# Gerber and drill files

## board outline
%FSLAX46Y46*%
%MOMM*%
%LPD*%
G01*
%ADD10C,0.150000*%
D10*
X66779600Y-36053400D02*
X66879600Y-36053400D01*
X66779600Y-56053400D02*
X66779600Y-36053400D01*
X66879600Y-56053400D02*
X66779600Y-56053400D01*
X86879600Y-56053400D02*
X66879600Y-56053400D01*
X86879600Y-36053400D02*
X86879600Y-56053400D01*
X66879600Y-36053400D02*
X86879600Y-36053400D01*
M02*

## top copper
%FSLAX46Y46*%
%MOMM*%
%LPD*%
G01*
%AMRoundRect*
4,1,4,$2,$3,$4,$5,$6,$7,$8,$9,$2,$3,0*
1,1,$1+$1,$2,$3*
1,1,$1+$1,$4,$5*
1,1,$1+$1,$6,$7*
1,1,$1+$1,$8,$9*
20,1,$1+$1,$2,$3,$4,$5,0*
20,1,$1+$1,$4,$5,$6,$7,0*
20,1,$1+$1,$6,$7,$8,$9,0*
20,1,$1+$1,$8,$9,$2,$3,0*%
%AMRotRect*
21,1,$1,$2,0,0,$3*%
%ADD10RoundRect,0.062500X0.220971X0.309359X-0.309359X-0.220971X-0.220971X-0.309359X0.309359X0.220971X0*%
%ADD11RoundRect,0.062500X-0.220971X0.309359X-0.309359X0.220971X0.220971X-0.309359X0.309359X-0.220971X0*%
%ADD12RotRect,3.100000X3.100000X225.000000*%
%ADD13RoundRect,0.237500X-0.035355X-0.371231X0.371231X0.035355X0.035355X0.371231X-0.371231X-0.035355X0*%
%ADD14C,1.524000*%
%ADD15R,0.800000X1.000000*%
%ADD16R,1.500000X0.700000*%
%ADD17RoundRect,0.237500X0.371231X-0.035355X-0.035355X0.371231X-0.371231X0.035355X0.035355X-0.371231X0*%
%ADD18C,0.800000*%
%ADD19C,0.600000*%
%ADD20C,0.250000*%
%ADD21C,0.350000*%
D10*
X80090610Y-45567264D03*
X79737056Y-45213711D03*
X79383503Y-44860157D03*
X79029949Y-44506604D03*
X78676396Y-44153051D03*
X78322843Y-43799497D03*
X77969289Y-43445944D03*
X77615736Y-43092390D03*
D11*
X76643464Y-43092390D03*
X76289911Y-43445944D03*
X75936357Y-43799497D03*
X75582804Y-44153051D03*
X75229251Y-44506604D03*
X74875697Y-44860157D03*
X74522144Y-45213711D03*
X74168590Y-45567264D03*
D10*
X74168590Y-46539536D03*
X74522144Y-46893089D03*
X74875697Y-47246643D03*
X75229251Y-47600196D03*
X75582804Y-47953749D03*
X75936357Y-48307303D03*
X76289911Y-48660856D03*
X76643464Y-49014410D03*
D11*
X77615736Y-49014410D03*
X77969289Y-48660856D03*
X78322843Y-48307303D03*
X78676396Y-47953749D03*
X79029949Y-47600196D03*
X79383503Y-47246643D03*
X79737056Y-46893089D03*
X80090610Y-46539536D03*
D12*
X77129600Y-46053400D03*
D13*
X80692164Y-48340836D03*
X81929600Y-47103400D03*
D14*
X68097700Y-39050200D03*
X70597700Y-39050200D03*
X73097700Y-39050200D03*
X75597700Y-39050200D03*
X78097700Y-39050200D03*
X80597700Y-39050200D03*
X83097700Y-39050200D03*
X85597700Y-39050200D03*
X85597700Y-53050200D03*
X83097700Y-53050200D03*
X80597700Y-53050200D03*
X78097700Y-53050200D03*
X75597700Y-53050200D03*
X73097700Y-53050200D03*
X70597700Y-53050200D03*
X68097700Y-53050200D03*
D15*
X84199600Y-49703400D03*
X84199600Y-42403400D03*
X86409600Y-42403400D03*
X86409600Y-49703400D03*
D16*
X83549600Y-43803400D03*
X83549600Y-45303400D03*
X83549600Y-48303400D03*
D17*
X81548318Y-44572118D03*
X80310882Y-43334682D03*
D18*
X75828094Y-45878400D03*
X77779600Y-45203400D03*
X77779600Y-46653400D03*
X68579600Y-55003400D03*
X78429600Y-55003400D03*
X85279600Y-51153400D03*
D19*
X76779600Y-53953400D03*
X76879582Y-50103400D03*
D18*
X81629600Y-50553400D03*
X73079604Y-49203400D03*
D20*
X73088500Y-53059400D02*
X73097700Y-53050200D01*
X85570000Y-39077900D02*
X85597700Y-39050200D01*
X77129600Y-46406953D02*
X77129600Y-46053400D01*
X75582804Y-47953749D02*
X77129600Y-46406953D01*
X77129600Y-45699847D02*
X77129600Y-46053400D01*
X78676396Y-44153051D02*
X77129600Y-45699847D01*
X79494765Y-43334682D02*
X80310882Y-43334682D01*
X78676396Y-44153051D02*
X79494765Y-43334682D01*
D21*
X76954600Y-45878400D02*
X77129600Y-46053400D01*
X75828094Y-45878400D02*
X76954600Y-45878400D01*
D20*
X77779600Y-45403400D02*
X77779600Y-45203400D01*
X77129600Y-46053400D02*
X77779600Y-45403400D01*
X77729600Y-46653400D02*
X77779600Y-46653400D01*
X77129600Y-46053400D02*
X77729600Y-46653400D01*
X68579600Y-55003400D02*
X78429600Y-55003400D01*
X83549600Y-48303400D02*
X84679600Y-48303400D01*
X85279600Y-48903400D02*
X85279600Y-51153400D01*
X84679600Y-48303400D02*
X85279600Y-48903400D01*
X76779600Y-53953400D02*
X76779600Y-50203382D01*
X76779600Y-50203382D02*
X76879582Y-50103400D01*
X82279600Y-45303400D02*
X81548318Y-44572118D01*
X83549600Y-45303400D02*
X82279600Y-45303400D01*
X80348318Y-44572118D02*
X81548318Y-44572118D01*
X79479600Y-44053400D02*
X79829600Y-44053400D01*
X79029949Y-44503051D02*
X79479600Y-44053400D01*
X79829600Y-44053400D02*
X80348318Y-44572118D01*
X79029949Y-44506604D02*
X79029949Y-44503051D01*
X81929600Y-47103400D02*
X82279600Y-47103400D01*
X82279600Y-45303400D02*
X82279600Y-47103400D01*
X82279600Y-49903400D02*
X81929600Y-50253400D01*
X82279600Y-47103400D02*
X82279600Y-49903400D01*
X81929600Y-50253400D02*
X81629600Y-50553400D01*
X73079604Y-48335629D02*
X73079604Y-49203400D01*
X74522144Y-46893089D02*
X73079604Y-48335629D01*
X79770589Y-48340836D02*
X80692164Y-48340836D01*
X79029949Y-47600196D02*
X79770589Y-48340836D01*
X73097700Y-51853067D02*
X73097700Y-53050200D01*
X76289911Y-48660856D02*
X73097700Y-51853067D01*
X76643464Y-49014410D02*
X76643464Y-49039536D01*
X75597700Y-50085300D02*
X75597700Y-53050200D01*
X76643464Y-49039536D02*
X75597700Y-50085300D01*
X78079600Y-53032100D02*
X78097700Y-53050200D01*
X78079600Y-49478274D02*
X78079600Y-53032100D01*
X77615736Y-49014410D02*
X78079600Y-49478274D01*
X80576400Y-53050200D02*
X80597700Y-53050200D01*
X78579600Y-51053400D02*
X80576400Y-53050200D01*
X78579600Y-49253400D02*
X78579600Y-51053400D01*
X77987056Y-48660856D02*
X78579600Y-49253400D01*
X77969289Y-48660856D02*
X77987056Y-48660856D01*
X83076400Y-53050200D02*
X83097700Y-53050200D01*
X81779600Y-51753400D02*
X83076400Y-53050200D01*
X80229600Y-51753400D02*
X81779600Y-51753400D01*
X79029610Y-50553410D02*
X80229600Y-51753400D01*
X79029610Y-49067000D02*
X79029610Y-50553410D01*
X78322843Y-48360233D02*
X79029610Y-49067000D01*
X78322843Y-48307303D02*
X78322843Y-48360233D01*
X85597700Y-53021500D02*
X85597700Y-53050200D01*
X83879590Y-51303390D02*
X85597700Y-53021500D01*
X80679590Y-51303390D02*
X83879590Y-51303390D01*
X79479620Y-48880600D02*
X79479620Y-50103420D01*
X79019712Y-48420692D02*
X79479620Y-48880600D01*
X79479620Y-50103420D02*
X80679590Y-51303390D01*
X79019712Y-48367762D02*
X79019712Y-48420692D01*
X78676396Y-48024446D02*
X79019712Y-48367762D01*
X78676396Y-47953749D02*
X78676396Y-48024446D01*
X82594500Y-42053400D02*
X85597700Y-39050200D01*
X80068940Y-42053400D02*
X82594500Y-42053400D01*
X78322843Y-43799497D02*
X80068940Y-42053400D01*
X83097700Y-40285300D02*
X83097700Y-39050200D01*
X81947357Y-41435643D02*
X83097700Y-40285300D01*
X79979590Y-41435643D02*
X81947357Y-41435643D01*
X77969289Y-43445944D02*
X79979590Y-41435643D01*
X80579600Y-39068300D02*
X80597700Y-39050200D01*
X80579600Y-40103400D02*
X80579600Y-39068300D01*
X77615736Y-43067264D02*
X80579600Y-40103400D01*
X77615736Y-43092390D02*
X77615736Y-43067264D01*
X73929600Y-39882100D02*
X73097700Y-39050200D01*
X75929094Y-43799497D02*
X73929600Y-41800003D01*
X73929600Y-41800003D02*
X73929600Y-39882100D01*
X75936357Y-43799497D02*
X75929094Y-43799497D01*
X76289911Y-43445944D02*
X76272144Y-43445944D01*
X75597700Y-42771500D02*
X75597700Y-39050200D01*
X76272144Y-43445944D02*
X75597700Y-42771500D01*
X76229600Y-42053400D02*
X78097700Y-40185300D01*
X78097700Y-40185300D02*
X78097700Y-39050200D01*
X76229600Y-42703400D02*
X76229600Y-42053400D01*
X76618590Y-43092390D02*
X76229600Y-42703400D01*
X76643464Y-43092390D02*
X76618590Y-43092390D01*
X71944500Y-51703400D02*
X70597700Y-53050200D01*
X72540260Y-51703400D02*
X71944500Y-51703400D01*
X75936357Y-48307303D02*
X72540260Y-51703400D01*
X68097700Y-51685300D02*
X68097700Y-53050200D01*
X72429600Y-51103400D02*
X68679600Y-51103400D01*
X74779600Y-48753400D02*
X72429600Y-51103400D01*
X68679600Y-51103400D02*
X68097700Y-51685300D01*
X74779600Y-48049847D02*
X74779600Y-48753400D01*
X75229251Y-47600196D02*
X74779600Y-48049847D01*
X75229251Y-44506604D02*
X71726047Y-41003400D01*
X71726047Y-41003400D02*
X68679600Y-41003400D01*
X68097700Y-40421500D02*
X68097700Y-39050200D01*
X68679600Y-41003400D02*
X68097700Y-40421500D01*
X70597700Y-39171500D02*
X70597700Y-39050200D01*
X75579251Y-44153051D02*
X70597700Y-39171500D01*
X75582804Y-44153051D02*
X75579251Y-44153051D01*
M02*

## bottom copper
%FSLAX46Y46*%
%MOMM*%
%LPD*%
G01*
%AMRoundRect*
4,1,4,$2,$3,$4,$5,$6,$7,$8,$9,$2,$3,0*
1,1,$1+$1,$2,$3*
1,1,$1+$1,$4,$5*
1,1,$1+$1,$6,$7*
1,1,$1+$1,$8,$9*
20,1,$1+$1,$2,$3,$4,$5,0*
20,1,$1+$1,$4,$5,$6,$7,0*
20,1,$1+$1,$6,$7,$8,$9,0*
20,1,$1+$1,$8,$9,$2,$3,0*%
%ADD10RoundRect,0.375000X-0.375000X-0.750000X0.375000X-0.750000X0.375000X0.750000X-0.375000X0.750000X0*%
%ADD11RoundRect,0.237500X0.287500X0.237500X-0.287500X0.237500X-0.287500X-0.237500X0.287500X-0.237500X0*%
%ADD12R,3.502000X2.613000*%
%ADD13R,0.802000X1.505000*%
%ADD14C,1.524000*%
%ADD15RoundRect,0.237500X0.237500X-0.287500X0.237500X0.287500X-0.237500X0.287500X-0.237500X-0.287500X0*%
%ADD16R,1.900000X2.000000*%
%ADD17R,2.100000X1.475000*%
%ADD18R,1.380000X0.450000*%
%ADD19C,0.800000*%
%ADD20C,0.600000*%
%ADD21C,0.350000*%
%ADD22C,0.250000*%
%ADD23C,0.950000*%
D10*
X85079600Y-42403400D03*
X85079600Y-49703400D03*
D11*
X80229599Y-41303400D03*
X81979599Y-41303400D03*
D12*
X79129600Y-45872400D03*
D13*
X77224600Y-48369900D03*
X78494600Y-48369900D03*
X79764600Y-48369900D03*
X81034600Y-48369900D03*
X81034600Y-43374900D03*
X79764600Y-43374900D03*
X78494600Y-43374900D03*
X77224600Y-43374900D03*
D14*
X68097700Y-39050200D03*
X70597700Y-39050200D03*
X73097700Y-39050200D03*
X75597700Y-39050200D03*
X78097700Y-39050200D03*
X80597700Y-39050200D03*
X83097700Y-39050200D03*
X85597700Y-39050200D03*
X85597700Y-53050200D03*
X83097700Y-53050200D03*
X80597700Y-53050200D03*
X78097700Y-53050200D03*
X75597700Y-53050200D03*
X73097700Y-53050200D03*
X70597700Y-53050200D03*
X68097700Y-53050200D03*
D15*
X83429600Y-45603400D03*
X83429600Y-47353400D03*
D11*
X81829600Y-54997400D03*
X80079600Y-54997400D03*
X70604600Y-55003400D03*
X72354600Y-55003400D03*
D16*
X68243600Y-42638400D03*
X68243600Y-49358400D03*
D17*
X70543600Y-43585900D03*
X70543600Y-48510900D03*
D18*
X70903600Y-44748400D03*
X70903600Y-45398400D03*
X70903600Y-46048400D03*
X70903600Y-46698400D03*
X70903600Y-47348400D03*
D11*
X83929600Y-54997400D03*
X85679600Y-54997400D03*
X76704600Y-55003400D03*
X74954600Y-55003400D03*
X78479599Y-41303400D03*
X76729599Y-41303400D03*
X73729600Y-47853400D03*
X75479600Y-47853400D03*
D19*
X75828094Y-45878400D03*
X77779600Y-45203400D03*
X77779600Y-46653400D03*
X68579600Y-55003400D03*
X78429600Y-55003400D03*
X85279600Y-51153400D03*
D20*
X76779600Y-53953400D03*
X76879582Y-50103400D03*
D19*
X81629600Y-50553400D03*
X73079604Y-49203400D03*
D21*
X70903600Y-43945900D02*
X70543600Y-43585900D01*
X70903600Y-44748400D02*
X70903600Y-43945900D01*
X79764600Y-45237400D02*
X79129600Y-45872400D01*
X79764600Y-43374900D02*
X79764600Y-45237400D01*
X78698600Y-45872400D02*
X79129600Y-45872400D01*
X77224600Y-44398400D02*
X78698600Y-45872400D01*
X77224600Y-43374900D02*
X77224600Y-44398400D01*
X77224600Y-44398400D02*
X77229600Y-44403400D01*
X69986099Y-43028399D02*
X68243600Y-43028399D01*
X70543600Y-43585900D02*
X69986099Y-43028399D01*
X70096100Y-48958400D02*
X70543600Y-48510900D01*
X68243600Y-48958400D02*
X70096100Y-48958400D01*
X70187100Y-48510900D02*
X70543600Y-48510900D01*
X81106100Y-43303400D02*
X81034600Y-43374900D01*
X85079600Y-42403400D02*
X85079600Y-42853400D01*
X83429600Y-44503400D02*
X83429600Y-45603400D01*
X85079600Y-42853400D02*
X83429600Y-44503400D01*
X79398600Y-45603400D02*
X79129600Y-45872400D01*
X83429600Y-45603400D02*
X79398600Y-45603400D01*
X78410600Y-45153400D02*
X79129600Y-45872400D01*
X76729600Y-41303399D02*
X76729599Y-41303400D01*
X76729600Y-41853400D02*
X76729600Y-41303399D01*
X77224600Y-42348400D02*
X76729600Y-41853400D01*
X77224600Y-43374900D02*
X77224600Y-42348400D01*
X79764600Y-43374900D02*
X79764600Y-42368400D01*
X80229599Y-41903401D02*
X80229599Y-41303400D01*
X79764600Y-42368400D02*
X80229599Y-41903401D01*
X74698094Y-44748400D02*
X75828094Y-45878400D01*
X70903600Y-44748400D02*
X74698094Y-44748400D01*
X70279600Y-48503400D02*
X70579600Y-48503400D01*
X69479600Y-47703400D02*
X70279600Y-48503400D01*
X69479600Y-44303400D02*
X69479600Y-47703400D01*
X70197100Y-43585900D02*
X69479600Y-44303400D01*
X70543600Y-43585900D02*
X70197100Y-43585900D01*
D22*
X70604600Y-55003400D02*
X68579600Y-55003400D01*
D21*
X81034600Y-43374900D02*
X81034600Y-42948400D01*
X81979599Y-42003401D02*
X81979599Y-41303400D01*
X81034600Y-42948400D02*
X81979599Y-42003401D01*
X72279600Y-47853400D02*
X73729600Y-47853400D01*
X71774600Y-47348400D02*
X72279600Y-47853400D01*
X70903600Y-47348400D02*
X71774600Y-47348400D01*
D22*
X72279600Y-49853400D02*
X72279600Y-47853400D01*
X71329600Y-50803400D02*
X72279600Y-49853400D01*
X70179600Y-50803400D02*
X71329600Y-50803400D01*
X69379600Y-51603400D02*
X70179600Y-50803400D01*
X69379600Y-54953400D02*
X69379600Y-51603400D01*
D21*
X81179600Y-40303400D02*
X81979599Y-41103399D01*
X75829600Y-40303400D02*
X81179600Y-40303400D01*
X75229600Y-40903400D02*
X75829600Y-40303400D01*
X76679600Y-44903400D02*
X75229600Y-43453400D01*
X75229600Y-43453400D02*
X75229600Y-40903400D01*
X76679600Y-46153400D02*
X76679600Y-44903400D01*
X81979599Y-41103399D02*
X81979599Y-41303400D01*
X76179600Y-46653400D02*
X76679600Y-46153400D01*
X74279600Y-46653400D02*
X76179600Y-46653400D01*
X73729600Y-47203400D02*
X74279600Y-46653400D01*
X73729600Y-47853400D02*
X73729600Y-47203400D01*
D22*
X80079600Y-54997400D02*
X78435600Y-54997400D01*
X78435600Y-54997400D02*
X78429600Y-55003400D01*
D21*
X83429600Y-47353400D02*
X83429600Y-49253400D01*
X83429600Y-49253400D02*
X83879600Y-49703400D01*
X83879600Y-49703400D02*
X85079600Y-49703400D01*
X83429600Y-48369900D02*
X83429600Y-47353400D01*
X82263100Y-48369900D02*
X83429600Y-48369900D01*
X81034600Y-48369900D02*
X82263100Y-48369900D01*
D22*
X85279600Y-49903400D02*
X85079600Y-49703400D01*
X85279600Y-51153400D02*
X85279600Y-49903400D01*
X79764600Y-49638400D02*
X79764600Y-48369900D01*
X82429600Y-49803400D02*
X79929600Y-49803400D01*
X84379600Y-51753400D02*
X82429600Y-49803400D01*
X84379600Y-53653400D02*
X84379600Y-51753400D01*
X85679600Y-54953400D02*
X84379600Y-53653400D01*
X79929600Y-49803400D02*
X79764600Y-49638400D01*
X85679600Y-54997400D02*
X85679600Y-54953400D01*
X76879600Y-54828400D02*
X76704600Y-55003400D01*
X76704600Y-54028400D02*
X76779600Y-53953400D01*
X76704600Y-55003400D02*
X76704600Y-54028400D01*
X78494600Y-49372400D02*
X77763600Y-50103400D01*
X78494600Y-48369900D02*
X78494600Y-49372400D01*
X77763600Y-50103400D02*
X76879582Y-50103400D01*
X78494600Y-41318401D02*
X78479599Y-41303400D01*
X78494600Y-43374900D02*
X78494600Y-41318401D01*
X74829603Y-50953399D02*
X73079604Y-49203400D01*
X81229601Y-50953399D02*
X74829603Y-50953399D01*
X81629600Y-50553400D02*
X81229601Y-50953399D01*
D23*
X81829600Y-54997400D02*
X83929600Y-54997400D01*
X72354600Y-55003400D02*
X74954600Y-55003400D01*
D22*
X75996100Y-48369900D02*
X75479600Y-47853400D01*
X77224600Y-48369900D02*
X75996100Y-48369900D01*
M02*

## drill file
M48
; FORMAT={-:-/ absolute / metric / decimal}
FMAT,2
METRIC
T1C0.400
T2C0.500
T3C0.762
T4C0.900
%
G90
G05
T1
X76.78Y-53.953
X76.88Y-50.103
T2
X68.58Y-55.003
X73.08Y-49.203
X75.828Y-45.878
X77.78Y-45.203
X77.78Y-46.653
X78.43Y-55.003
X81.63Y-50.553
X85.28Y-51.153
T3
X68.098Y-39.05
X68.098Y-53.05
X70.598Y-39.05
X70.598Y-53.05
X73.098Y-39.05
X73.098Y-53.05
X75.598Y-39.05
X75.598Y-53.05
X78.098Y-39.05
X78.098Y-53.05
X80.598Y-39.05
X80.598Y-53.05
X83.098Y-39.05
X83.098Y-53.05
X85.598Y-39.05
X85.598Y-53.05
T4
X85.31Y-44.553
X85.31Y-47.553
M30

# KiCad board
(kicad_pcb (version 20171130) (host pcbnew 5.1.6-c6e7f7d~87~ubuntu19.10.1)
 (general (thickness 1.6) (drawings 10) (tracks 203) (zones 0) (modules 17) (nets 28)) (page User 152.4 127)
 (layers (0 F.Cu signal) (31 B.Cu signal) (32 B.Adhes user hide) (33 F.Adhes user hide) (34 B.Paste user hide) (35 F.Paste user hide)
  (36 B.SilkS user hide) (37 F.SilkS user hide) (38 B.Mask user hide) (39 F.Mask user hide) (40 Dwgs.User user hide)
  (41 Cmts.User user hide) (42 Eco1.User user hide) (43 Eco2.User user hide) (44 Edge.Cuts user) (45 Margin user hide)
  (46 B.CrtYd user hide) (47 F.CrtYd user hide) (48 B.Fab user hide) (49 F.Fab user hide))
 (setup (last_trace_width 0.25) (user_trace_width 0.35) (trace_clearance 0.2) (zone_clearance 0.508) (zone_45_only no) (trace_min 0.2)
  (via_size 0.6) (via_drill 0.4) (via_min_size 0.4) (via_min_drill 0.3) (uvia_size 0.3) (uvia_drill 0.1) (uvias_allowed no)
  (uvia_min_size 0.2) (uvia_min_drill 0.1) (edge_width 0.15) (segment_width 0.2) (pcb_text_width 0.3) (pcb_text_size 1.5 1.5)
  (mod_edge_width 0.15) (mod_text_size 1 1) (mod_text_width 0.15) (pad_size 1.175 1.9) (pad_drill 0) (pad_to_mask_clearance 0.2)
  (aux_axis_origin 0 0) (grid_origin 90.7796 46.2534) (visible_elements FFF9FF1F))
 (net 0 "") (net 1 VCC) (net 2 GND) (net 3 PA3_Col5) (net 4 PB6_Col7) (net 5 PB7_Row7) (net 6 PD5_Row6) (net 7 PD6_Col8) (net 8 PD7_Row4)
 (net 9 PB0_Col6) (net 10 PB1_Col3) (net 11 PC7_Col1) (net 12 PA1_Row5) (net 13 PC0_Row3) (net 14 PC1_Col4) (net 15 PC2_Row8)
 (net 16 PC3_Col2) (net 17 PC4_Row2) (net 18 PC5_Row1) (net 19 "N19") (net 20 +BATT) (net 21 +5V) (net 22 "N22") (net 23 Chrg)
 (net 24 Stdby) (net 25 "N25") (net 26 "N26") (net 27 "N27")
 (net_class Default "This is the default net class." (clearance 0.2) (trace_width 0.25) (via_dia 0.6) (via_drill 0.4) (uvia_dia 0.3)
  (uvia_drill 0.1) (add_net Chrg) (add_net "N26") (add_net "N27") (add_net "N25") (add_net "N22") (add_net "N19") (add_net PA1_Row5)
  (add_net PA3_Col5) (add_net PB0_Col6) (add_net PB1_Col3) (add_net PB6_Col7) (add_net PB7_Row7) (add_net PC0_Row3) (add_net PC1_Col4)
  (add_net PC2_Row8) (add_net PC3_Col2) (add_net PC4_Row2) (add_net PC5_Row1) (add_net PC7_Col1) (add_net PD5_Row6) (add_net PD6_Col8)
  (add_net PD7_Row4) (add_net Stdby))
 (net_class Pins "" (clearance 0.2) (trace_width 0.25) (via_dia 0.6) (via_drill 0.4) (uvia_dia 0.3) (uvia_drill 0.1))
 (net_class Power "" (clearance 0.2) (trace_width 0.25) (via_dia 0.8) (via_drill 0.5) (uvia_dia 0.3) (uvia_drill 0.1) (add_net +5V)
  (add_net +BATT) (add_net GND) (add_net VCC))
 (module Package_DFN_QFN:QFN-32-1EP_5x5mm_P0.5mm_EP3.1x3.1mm (layer F.Cu) (at 77.1296 46.0534 225)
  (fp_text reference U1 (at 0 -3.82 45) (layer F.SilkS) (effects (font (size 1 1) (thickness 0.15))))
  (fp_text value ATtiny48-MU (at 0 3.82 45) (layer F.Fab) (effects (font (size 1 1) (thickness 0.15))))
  (pad 1 smd roundrect (at -2.4375 -1.75 225) (size 0.875 0.25) (layers F.Cu F.Paste F.Mask) (roundrect_rratio 0.25))
  (pad 2 smd roundrect (at -2.4375 -1.25 225) (size 0.875 0.25) (layers F.Cu F.Paste F.Mask) (roundrect_rratio 0.25))
  (pad 3 smd roundrect (at -2.4375 -0.75 225) (size 0.875 0.25) (layers F.Cu F.Paste F.Mask) (roundrect_rratio 0.25))
  (pad 4 smd roundrect (at -2.4375 -0.25 225) (size 0.875 0.25) (layers F.Cu F.Paste F.Mask) (roundrect_rratio 0.25) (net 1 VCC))
  (pad 5 smd roundrect (at -2.4375 0.25 225) (size 0.875 0.25) (layers F.Cu F.Paste F.Mask) (roundrect_rratio 0.25) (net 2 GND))
  (pad 6 smd roundrect (at -2.4375 0.75 225) (size 0.875 0.25) (layers F.Cu F.Paste F.Mask) (roundrect_rratio 0.25) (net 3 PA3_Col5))
  (pad 7 smd roundrect (at -2.4375 1.25 225) (size 0.875 0.25) (layers F.Cu F.Paste F.Mask) (roundrect_rratio 0.25) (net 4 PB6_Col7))
  (pad 8 smd roundrect (at -2.4375 1.75 225) (size 0.875 0.25) (layers F.Cu F.Paste F.Mask) (roundrect_rratio 0.25) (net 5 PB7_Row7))
  (pad 9 smd roundrect (at -1.75 2.4375 225) (size 0.25 0.875) (layers F.Cu F.Paste F.Mask) (roundrect_rratio 0.25) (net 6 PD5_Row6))
  (pad 10 smd roundrect (at -1.25 2.4375 225) (size 0.25 0.875) (layers F.Cu F.Paste F.Mask) (roundrect_rratio 0.25) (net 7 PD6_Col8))
  (pad 11 smd roundrect (at -0.75 2.4375 225) (size 0.25 0.875) (layers F.Cu F.Paste F.Mask) (roundrect_rratio 0.25) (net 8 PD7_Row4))
  (pad 12 smd roundrect (at -0.25 2.4375 225) (size 0.25 0.875) (layers F.Cu F.Paste F.Mask) (roundrect_rratio 0.25) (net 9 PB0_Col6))
  (pad 13 smd roundrect (at 0.25 2.4375 225) (size 0.25 0.875) (layers F.Cu F.Paste F.Mask) (roundrect_rratio 0.25) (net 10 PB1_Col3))
  (pad 14 smd roundrect (at 0.75 2.4375 225) (size 0.25 0.875) (layers F.Cu F.Paste F.Mask) (roundrect_rratio 0.25))
  (pad 15 smd roundrect (at 1.25 2.4375 225) (size 0.25 0.875) (layers F.Cu F.Paste F.Mask) (roundrect_rratio 0.25))
  (pad 16 smd roundrect (at 1.75 2.4375 225) (size 0.25 0.875) (layers F.Cu F.Paste F.Mask) (roundrect_rratio 0.25))
  (pad 17 smd roundrect (at 2.4375 1.75 225) (size 0.875 0.25) (layers F.Cu F.Paste F.Mask) (roundrect_rratio 0.25))
  (pad 18 smd roundrect (at 2.4375 1.25 225) (size 0.875 0.25) (layers F.Cu F.Paste F.Mask) (roundrect_rratio 0.25) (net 1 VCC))
  (pad 19 smd roundrect (at 2.4375 0.75 225) (size 0.875 0.25) (layers F.Cu F.Paste F.Mask) (roundrect_rratio 0.25))
  (pad 20 smd roundrect (at 2.4375 0.25 225) (size 0.875 0.25) (layers F.Cu F.Paste F.Mask) (roundrect_rratio 0.25) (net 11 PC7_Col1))
  (pad 21 smd roundrect (at 2.4375 -0.25 225) (size 0.875 0.25) (layers F.Cu F.Paste F.Mask) (roundrect_rratio 0.25) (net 2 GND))
  (pad 22 smd roundrect (at 2.4375 -0.75 225) (size 0.875 0.25) (layers F.Cu F.Paste F.Mask) (roundrect_rratio 0.25) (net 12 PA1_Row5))
  (pad 23 smd roundrect (at 2.4375 -1.25 225) (size 0.875 0.25) (layers F.Cu F.Paste F.Mask) (roundrect_rratio 0.25) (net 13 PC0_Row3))
  (pad 24 smd roundrect (at 2.4375 -1.75 225) (size 0.875 0.25) (layers F.Cu F.Paste F.Mask) (roundrect_rratio 0.25) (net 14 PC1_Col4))
  (pad 25 smd roundrect (at 1.75 -2.4375 225) (size 0.25 0.875) (layers F.Cu F.Paste F.Mask) (roundrect_rratio 0.25) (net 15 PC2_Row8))
  (pad 26 smd roundrect (at 1.25 -2.4375 225) (size 0.25 0.875) (layers F.Cu F.Paste F.Mask) (roundrect_rratio 0.25) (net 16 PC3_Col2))
  (pad 27 smd roundrect (at 0.75 -2.4375 225) (size 0.25 0.875) (layers F.Cu F.Paste F.Mask) (roundrect_rratio 0.25) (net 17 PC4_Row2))
  (pad 28 smd roundrect (at 0.25 -2.4375 225) (size 0.25 0.875) (layers F.Cu F.Paste F.Mask) (roundrect_rratio 0.25) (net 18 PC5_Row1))
  (pad 29 smd roundrect (at -0.25 -2.4375 225) (size 0.25 0.875) (layers F.Cu F.Paste F.Mask) (roundrect_rratio 0.25) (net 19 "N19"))
  (pad 30 smd roundrect (at -0.75 -2.4375 225) (size 0.25 0.875) (layers F.Cu F.Paste F.Mask) (roundrect_rratio 0.25))
  (pad 31 smd roundrect (at -1.25 -2.4375 225) (size 0.25 0.875) (layers F.Cu F.Paste F.Mask) (roundrect_rratio 0.25))
  (pad 32 smd roundrect (at -1.75 -2.4375 225) (size 0.25 0.875) (layers F.Cu F.Paste F.Mask) (roundrect_rratio 0.25))
  (pad 33 smd rect (at 0 0 225) (size 3.1 3.1) (layers F.Cu F.Mask) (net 2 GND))
  (pad "" smd roundrect (at -1.03 -1.03 225) (size 0.83 0.83) (layers F.Paste) (roundrect_rratio 0.25))
  (pad "" smd roundrect (at -1.03 0 225) (size 0.83 0.83) (layers F.Paste) (roundrect_rratio 0.25))
  (pad "" smd roundrect (at -1.03 1.03 225) (size 0.83 0.83) (layers F.Paste) (roundrect_rratio 0.25))
  (pad "" smd roundrect (at 0 -1.03 225) (size 0.83 0.83) (layers F.Paste) (roundrect_rratio 0.25))
  (pad "" smd roundrect (at 0 0 225) (size 0.83 0.83) (layers F.Paste) (roundrect_rratio 0.25))
  (pad "" smd roundrect (at 0 1.03 225) (size 0.83 0.83) (layers F.Paste) (roundrect_rratio 0.25))
  (pad "" smd roundrect (at 1.03 -1.03 225) (size 0.83 0.83) (layers F.Paste) (roundrect_rratio 0.25))
  (pad "" smd roundrect (at 1.03 0 225) (size 0.83 0.83) (layers F.Paste) (roundrect_rratio 0.25))
  (pad "" smd roundrect (at 1.03 1.03 225) (size 0.83 0.83) (layers F.Paste) (roundrect_rratio 0.25)))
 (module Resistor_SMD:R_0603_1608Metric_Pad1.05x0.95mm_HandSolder (layer F.Cu) (at 81.310882 47.722118 45)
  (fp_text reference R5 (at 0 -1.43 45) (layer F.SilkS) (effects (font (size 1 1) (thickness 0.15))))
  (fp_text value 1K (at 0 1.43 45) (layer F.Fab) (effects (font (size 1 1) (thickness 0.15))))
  (pad 1 smd roundrect (at -0.875 0 45) (size 1.05 0.95) (layers F.Cu F.Paste F.Mask) (roundrect_rratio 0.25) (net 19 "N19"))
  (pad 2 smd roundrect (at 0.875 0 45) (size 1.05 0.95) (layers F.Cu F.Paste F.Mask) (roundrect_rratio 0.25) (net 1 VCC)))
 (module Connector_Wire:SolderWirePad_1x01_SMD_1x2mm (layer B.Cu) (at 85.0796 42.4034)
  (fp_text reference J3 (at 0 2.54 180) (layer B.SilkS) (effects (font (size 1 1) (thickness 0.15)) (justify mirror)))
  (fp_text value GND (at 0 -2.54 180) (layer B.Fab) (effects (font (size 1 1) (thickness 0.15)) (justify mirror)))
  (pad 1 smd roundrect (at 0 0) (size 1.5 2.25) (layers B.Cu B.Paste B.Mask) (roundrect_rratio 0.25) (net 2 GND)))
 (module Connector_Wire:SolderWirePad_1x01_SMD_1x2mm (layer B.Cu) (at 85.0796 49.7034)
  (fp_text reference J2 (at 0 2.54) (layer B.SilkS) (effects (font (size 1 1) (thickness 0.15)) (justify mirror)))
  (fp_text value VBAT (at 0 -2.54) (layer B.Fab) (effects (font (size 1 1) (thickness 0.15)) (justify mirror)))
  (pad 1 smd roundrect (at 0 0) (size 1.5 2.25) (layers B.Cu B.Paste B.Mask) (roundrect_rratio 0.25) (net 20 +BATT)))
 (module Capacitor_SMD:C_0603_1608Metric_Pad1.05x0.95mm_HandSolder (layer B.Cu) (at 81.104599 41.3034 180)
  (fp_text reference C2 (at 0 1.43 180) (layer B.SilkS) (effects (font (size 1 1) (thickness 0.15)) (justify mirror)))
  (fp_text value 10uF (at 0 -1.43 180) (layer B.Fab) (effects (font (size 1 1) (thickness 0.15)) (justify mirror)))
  (pad 2 smd roundrect (at 0.875 0 180) (size 1.05 0.95) (layers B.Cu B.Paste B.Mask) (roundrect_rratio 0.25) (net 2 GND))
  (pad 1 smd roundrect (at -0.875 0 180) (size 1.05 0.95) (layers B.Cu B.Paste B.Mask) (roundrect_rratio 0.25) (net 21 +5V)))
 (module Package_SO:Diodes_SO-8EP (layer B.Cu) (at 79.1296 45.8724 270)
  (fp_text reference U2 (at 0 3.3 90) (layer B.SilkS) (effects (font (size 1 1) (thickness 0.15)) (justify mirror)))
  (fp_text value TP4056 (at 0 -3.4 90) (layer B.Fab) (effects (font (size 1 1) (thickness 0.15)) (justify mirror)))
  (pad 9 smd rect (at 0 0 270) (size 2.613 3.502) (layers B.Cu B.Paste B.Mask) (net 2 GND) (solder_paste_margin_ratio -0.2))
  (pad 8 smd rect (at 2.4975 1.905 270) (size 1.505 0.802) (layers B.Cu B.Paste B.Mask) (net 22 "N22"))
  (pad 7 smd rect (at 2.4975 0.635 270) (size 1.505 0.802) (layers B.Cu B.Paste B.Mask) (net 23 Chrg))
  (pad 6 smd rect (at 2.4975 -0.635 270) (size 1.505 0.802) (layers B.Cu B.Paste B.Mask) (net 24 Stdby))
  (pad 5 smd rect (at 2.4975 -1.905 270) (size 1.505 0.802) (layers B.Cu B.Paste B.Mask) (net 20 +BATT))
  (pad 4 smd rect (at -2.4975 -1.905 270) (size 1.505 0.802) (layers B.Cu B.Paste B.Mask) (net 21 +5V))
  (pad 3 smd rect (at -2.4975 -0.635 270) (size 1.505 0.802) (layers B.Cu B.Paste B.Mask) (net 2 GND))
  (pad 2 smd rect (at -2.4975 0.635 270) (size 1.505 0.802) (layers B.Cu B.Paste B.Mask) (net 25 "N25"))
  (pad 1 smd rect (at -2.4975 1.905 270) (size 1.505 0.802) (layers B.Cu B.Paste B.Mask) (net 2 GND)))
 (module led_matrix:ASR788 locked (layer F.Cu) (at 76.8477 46.0502)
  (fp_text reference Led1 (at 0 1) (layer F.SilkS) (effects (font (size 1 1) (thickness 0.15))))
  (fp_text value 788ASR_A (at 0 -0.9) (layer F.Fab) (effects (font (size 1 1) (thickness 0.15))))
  (pad 16 thru_hole circle (at -8.75 -7) (size 1.524 1.524) (drill 0.762) (layers *.Cu *.Mask) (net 10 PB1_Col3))
  (pad 15 thru_hole circle (at -6.25 -7) (size 1.524 1.524) (drill 0.762) (layers *.Cu *.Mask) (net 9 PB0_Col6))
  (pad 14 thru_hole circle (at -3.75 -7) (size 1.524 1.524) (drill 0.762) (layers *.Cu *.Mask) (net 8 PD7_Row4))
  (pad 13 thru_hole circle (at -1.25 -7) (size 1.524 1.524) (drill 0.762) (layers *.Cu *.Mask) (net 7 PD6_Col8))
  (pad 12 thru_hole circle (at 1.25 -7) (size 1.524 1.524) (drill 0.762) (layers *.Cu *.Mask) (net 6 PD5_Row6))
  (pad 11 thru_hole circle (at 3.75 -7) (size 1.524 1.524) (drill 0.762) (layers *.Cu *.Mask) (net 5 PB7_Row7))
  (pad 10 thru_hole circle (at 6.25 -7) (size 1.524 1.524) (drill 0.762) (layers *.Cu *.Mask) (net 4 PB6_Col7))
  (pad 9 thru_hole circle (at 8.75 -7) (size 1.524 1.524) (drill 0.762) (layers *.Cu *.Mask) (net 3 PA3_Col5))
  (pad 8 thru_hole circle (at 8.75 7) (size 1.524 1.524) (drill 0.762) (layers *.Cu *.Mask) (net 18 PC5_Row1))
  (pad 7 thru_hole circle (at 6.25 7) (size 1.524 1.524) (drill 0.762) (layers *.Cu *.Mask) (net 17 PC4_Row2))
  (pad 6 thru_hole circle (at 3.75 7) (size 1.524 1.524) (drill 0.762) (layers *.Cu *.Mask) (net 16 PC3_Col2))
  (pad 5 thru_hole circle (at 1.25 7) (size 1.524 1.524) (drill 0.762) (layers *.Cu *.Mask) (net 15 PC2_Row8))
  (pad 4 thru_hole circle (at -1.25 7) (size 1.524 1.524) (drill 0.762) (layers *.Cu *.Mask) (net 14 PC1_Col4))
  (pad 3 thru_hole circle (at -3.75 7) (size 1.524 1.524) (drill 0.762) (layers *.Cu *.Mask) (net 13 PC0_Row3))
  (pad 2 thru_hole circle (at -6.25 7) (size 1.524 1.524) (drill 0.762) (layers *.Cu *.Mask) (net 12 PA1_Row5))
  (pad 1 thru_hole circle (at -8.75 7) (size 1.524 1.524) (drill 0.762) (layers *.Cu *.Mask) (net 11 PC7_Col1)))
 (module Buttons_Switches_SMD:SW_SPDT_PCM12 (layer F.Cu) (at 84.9796 46.0534 90)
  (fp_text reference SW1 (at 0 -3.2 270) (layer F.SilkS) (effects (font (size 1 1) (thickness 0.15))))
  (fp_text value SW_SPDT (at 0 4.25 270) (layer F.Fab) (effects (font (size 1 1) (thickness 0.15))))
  (pad "" smd rect (at -3.65 -0.78 90) (size 1 0.8) (layers F.Cu F.Paste F.Mask))
  (pad "" smd rect (at 3.65 -0.78 90) (size 1 0.8) (layers F.Cu F.Paste F.Mask))
  (pad "" smd rect (at 3.65 1.43 90) (size 1 0.8) (layers F.Cu F.Paste F.Mask))
  (pad "" smd rect (at -3.65 1.43 90) (size 1 0.8) (layers F.Cu F.Paste F.Mask))
  (pad 3 smd rect (at 2.25 -1.43 90) (size 0.7 1.5) (layers F.Cu F.Paste F.Mask))
  (pad 2 smd rect (at 0.75 -1.43 90) (size 0.7 1.5) (layers F.Cu F.Paste F.Mask) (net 1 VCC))
  (pad 1 smd rect (at -2.25 -1.43 90) (size 0.7 1.5) (layers F.Cu F.Paste F.Mask) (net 20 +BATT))
  (pad "" np_thru_hole circle (at 1.5 0.33 90) (size 0.9 0.9) (drill 0.9) (layers *.Cu *.Mask))
  (pad "" np_thru_hole circle (at -1.5 0.33 90) (size 0.9 0.9) (drill 0.9) (layers *.Cu *.Mask)))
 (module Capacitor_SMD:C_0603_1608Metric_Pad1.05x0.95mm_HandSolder (layer F.Cu) (at 80.9296 43.9534 135)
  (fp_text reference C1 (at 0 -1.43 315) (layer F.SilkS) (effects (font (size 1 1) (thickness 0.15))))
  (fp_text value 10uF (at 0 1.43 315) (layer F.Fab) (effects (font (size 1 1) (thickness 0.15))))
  (pad 1 smd roundrect (at -0.875 0 135) (size 1.05 0.95) (layers F.Cu F.Paste F.Mask) (roundrect_rratio 0.25) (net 1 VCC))
  (pad 2 smd roundrect (at 0.875 0 135) (size 1.05 0.95) (layers F.Cu F.Paste F.Mask) (roundrect_rratio 0.25) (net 2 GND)))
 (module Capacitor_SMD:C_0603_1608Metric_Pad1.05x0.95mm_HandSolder (layer B.Cu) (at 83.4296 46.4784 90)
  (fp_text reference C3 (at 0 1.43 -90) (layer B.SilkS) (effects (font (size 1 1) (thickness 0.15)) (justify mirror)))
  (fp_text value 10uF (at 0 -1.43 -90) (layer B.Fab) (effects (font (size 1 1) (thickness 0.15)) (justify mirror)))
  (pad 2 smd roundrect (at 0.875 0 90) (size 1.05 0.95) (layers B.Cu B.Paste B.Mask) (roundrect_rratio 0.25) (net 2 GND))
  (pad 1 smd roundrect (at -0.875 0 90) (size 1.05 0.95) (layers B.Cu B.Paste B.Mask) (roundrect_rratio 0.25) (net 20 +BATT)))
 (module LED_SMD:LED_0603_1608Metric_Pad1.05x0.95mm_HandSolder (layer B.Cu) (at 80.9546 54.9974 180)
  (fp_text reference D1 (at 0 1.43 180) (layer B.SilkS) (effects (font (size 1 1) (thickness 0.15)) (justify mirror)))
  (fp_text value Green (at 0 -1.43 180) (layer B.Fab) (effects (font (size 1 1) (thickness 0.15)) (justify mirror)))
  (pad 1 smd roundrect (at -0.875 0 180) (size 1.05 0.95) (layers B.Cu B.Paste B.Mask) (roundrect_rratio 0.25) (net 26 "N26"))
  (pad 2 smd roundrect (at 0.875 0 180) (size 1.05 0.95) (layers B.Cu B.Paste B.Mask) (roundrect_rratio 0.25) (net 21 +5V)))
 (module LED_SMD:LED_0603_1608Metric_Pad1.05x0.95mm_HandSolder (layer B.Cu) (at 71.4796 55.0034 180)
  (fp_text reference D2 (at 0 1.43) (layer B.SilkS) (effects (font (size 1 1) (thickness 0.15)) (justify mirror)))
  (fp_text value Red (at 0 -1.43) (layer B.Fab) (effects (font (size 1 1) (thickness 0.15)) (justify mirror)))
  (pad 2 smd roundrect (at 0.875 0 180) (size 1.05 0.95) (layers B.Cu B.Paste B.Mask) (roundrect_rratio 0.25) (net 21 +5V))
  (pad 1 smd roundrect (at -0.875 0 180) (size 1.05 0.95) (layers B.Cu B.Paste B.Mask) (roundrect_rratio 0.25) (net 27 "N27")))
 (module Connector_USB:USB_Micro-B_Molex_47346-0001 (layer B.Cu) (at 69.4436 46.0484 90)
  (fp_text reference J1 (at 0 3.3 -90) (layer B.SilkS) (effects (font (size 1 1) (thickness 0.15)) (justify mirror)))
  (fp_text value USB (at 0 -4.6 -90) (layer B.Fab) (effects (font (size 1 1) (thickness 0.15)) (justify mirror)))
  (pad 6 smd rect (at 0.84 -1.2 90) (size 1.175 1.9) (layers Eco1.User))
  (pad 6 smd rect (at -0.84 -1.2 90) (size 1.175 1.9) (layers Eco1.User))
  (pad 6 smd rect (at 3.41 -1.2 90) (size 2 1.9) (layers B.Cu B.Paste B.Mask) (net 2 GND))
  (pad 6 smd rect (at -3.31 -1.2 90) (size 2 1.9) (layers B.Cu B.Paste B.Mask) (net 2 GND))
  (pad 6 smd rect (at 2.4625 1.1 90) (size 1.475 2.1) (layers B.Cu B.Paste B.Mask) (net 2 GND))
  (pad 6 smd rect (at -2.4625 1.1 90) (size 1.475 2.1) (layers B.Cu B.Paste B.Mask) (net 2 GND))
  (pad 5 smd rect (at 1.3 1.46 90) (size 0.45 1.38) (layers B.Cu B.Paste B.Mask) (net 2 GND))
  (pad 4 smd rect (at 0.65 1.46 90) (size 0.45 1.38) (layers B.Cu B.Paste B.Mask))
  (pad 3 smd rect (at 0 1.46 90) (size 0.45 1.38) (layers B.Cu B.Paste B.Mask))
  (pad 2 smd rect (at -0.65 1.46 90) (size 0.45 1.38) (layers B.Cu B.Paste B.Mask))
  (pad 1 smd rect (at -1.3 1.46 90) (size 0.45 1.38) (layers B.Cu B.Paste B.Mask) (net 21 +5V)))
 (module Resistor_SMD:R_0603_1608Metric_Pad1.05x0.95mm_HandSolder (layer B.Cu) (at 84.8046 54.9974 180)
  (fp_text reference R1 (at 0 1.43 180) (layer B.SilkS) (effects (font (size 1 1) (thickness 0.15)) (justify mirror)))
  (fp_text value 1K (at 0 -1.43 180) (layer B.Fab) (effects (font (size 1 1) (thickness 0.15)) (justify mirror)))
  (pad 2 smd roundrect (at 0.875 0 180) (size 1.05 0.95) (layers B.Cu B.Paste B.Mask) (roundrect_rratio 0.25) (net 26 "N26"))
  (pad 1 smd roundrect (at -0.875 0 180) (size 1.05 0.95) (layers B.Cu B.Paste B.Mask) (roundrect_rratio 0.25) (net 24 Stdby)))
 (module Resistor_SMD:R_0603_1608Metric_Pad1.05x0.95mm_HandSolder (layer B.Cu) (at 75.8296 55.0034 180)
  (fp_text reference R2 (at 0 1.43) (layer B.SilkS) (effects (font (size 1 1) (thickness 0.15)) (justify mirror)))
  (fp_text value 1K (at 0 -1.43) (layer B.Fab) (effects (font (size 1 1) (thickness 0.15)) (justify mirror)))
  (pad 1 smd roundrect (at -0.875 0 180) (size 1.05 0.95) (layers B.Cu B.Paste B.Mask) (roundrect_rratio 0.25) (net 23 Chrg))
  (pad 2 smd roundrect (at 0.875 0 180) (size 1.05 0.95) (layers B.Cu B.Paste B.Mask) (roundrect_rratio 0.25) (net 27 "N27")))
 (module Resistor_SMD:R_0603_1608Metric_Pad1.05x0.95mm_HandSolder (layer B.Cu) (at 77.604599 41.3034 180)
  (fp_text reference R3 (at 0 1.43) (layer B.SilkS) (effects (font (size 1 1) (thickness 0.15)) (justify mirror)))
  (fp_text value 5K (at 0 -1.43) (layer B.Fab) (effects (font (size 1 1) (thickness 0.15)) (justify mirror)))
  (pad 1 smd roundrect (at -0.875 0 180) (size 1.05 0.95) (layers B.Cu B.Paste B.Mask) (roundrect_rratio 0.25) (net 25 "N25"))
  (pad 2 smd roundrect (at 0.875 0 180) (size 1.05 0.95) (layers B.Cu B.Paste B.Mask) (roundrect_rratio 0.25) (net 2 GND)))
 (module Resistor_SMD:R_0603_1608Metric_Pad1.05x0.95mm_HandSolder (layer B.Cu) (at 74.6046 47.8534 180)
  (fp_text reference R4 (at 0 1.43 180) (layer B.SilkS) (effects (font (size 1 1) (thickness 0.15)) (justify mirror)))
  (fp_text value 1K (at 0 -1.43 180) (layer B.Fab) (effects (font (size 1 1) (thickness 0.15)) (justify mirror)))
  (pad 2 smd roundrect (at 0.875 0 180) (size 1.05 0.95) (layers B.Cu B.Paste B.Mask) (roundrect_rratio 0.25) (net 21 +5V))
  (pad 1 smd roundrect (at -0.875 0 180) (size 1.05 0.95) (layers B.Cu B.Paste B.Mask) (roundrect_rratio 0.25) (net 22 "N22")))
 (gr_line (start 66.7796 36.0534) (end 66.8796 36.0534) (layer Edge.Cuts) (width 0.15))
 (gr_line (start 66.7796 56.0534) (end 66.7796 36.0534) (layer Edge.Cuts) (width 0.15))
 (gr_line (start 66.8796 56.0534) (end 66.7796 56.0534) (layer Edge.Cuts) (width 0.15))
 (gr_line (start 86.8796 56.0534) (end 66.8796 56.0534) (layer Edge.Cuts) (width 0.15))
 (gr_line (start 86.8796 36.0534) (end 86.8796 56.0534) (layer Edge.Cuts) (width 0.15))
 (gr_line (start 66.8796 36.0534) (end 86.8796 36.0534) (layer Edge.Cuts) (width 0.15))
 (segment (start 70.9036 43.9459) (end 70.5436 43.5859) (width 0.35) (layer B.Cu) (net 2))
 (segment (start 70.9036 44.7484) (end 70.9036 43.9459) (width 0.35) (layer B.Cu) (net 2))
 (segment (start 79.7646 45.2374) (end 79.1296 45.8724) (width 0.35) (layer B.Cu) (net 2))
 (segment (start 79.7646 43.3749) (end 79.7646 45.2374) (width 0.35) (layer B.Cu) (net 2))
 (segment (start 78.6986 45.8724) (end 79.1296 45.8724) (width 0.35) (layer B.Cu) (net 2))
 (segment (start 77.2246 44.3984) (end 78.6986 45.8724) (width 0.35) (layer B.Cu) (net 2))
 (segment (start 77.2246 43.3749) (end 77.2246 44.3984) (width 0.35) (layer B.Cu) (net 2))
 (segment (start 77.2246 44.3984) (end 77.2296 44.4034) (width 0.35) (layer B.Cu) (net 2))
 (segment (start 69.986099 43.028399) (end 68.2436 43.028399) (width 0.35) (layer B.Cu) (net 2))
 (segment (start 70.5436 43.5859) (end 69.986099 43.028399) (width 0.35) (layer B.Cu) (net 2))
 (segment (start 70.0961 48.9584) (end 70.5436 48.5109) (width 0.35) (layer B.Cu) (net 2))
 (segment (start 68.2436 48.9584) (end 70.0961 48.9584) (width 0.35) (layer B.Cu) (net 2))
 (segment (start 70.1871 48.5109) (end 70.5436 48.5109) (width 0.35) (layer B.Cu) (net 2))
 (segment (start 81.1061 43.3034) (end 81.0346 43.3749) (width 0.35) (layer B.Cu) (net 21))
 (segment (start 73.0885 53.0594) (end 73.0977 53.0502) (width 0.25) (layer F.Cu) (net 13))
 (segment (start 85.57 39.0779) (end 85.5977 39.0502) (width 0.25) (layer F.Cu) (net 3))
 (segment (start 85.0796 42.4034) (end 85.0796 42.8534) (width 0.35) (layer B.Cu) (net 2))
 (segment (start 83.4296 44.5034) (end 83.4296 45.6034) (width 0.35) (layer B.Cu) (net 2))
 (segment (start 85.0796 42.8534) (end 83.4296 44.5034) (width 0.35) (layer B.Cu) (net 2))
 (segment (start 79.3986 45.6034) (end 79.1296 45.8724) (width 0.35) (layer B.Cu) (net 2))
 (segment (start 83.4296 45.6034) (end 79.3986 45.6034) (width 0.35) (layer B.Cu) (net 2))
 (segment (start 78.4106 45.1534) (end 79.1296 45.8724) (width 0.35) (layer B.Cu) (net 2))
 (segment (start 77.1296 46.406953) (end 77.1296 46.0534) (width 0.25) (layer F.Cu) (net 2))
 (segment (start 75.582804 47.953749) (end 77.1296 46.406953) (width 0.25) (layer F.Cu) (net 2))
 (segment (start 77.1296 45.699847) (end 77.1296 46.0534) (width 0.25) (layer F.Cu) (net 2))
 (segment (start 78.676396 44.153051) (end 77.1296 45.699847) (width 0.25) (layer F.Cu) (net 2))
 (segment (start 79.494765 43.334682) (end 80.310882 43.334682) (width 0.25) (layer F.Cu) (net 2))
 (segment (start 78.676396 44.153051) (end 79.494765 43.334682) (width 0.25) (layer F.Cu) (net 2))
 (segment (start 76.7296 41.303399) (end 76.729599 41.3034) (width 0.35) (layer B.Cu) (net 2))
 (segment (start 76.7296 41.8534) (end 76.7296 41.303399) (width 0.35) (layer B.Cu) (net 2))
 (segment (start 77.2246 42.3484) (end 76.7296 41.8534) (width 0.35) (layer B.Cu) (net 2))
 (segment (start 77.2246 43.3749) (end 77.2246 42.3484) (width 0.35) (layer B.Cu) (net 2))
 (segment (start 79.7646 43.3749) (end 79.7646 42.3684) (width 0.35) (layer B.Cu) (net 2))
 (segment (start 80.229599 41.903401) (end 80.229599 41.3034) (width 0.35) (layer B.Cu) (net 2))
 (segment (start 79.7646 42.3684) (end 80.229599 41.903401) (width 0.35) (layer B.Cu) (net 2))
 (segment (start 74.698094 44.7484) (end 75.828094 45.8784) (width 0.35) (layer B.Cu) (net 2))
 (via (at 75.828094 45.8784) (size 0.8) (drill 0.5) (layers F.Cu B.Cu) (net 2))
 (segment (start 70.9036 44.7484) (end 74.698094 44.7484) (width 0.35) (layer B.Cu) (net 2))
 (segment (start 76.9546 45.8784) (end 77.1296 46.0534) (width 0.35) (layer F.Cu) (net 2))
 (segment (start 75.828094 45.8784) (end 76.9546 45.8784) (width 0.35) (layer F.Cu) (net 2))
 (segment (start 77.7796 45.4034) (end 77.7796 45.2034) (width 0.25) (layer F.Cu) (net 2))
 (segment (start 77.1296 46.0534) (end 77.7796 45.4034) (width 0.25) (layer F.Cu) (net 2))
 (via (at 77.7796 45.2034) (size 0.8) (drill 0.5) (layers F.Cu B.Cu) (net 2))
 (segment (start 77.7296 46.6534) (end 77.7796 46.6534) (width 0.25) (layer F.Cu) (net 2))
 (segment (start 77.1296 46.0534) (end 77.7296 46.6534) (width 0.25) (layer F.Cu) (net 2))
 (via (at 77.7796 46.6534) (size 0.8) (drill 0.5) (layers F.Cu B.Cu) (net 2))
 (segment (start 70.2796 48.5034) (end 70.5796 48.5034) (width 0.35) (layer B.Cu) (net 2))
 (segment (start 69.4796 47.7034) (end 70.2796 48.5034) (width 0.35) (layer B.Cu) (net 2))
 (segment (start 69.4796 44.3034) (end 69.4796 47.7034) (width 0.35) (layer B.Cu) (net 2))
 (segment (start 70.1971 43.5859) (end 69.4796 44.3034) (width 0.35) (layer B.Cu) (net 2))
 (segment (start 70.5436 43.5859) (end 70.1971 43.5859) (width 0.35) (layer B.Cu) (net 2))
 (via (at 68.5796 55.0034) (size 0.8) (drill 0.5) (layers F.Cu B.Cu) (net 21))
 (segment (start 70.6046 55.0034) (end 68.5796 55.0034) (width 0.25) (layer B.Cu) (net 21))
 (segment (start 81.0346 43.3749) (end 81.0346 42.9484) (width 0.35) (layer B.Cu) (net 21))
 (segment (start 81.979599 42.003401) (end 81.979599 41.3034) (width 0.35) (layer B.Cu) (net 21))
 (segment (start 81.0346 42.9484) (end 81.979599 42.003401) (width 0.35) (layer B.Cu) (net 21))
 (segment (start 72.2796 47.8534) (end 73.7296 47.8534) (width 0.35) (layer B.Cu) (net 21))
 (segment (start 71.7746 47.3484) (end 72.2796 47.8534) (width 0.35) (layer B.Cu) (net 21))
 (segment (start 70.9036 47.3484) (end 71.7746 47.3484) (width 0.35) (layer B.Cu) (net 21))
 (segment (start 72.2796 49.8534) (end 72.2796 47.8534) (width 0.25) (layer B.Cu) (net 21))
 (segment (start 71.3296 50.8034) (end 72.2796 49.8534) (width 0.25) (layer B.Cu) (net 21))
 (segment (start 70.1796 50.8034) (end 71.3296 50.8034) (width 0.25) (layer B.Cu) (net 21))
 (segment (start 69.3796 51.6034) (end 70.1796 50.8034) (width 0.25) (layer B.Cu) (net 21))
 (segment (start 69.3796 54.9534) (end 69.3796 51.6034) (width 0.25) (layer B.Cu) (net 21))
 (segment (start 81.1796 40.3034) (end 81.979599 41.103399) (width 0.35) (layer B.Cu) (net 21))
 (segment (start 75.8296 40.3034) (end 81.1796 40.3034) (width 0.35) (layer B.Cu) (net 21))
 (segment (start 75.2296 40.9034) (end 75.8296 40.3034) (width 0.35) (layer B.Cu) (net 21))
 (segment (start 76.6796 44.9034) (end 75.2296 43.4534) (width 0.35) (layer B.Cu) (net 21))
 (segment (start 75.2296 43.4534) (end 75.2296 40.9034) (width 0.35) (layer B.Cu) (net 21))
 (segment (start 76.6796 46.1534) (end 76.6796 44.9034) (width 0.35) (layer B.Cu) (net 21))
 (segment (start 81.979599 41.103399) (end 81.979599 41.3034) (width 0.35) (layer B.Cu) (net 21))
 (segment (start 76.1796 46.6534) (end 76.6796 46.1534) (width 0.35) (layer B.Cu) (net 21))
 (segment (start 74.2796 46.6534) (end 76.1796 46.6534) (width 0.35) (layer B.Cu) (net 21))
 (segment (start 73.7296 47.2034) (end 74.2796 46.6534) (width 0.35) (layer B.Cu) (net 21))
 (segment (start 73.7296 47.8534) (end 73.7296 47.2034) (width 0.35) (layer B.Cu) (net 21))
 (segment (start 68.5796 55.0034) (end 78.4296 55.0034) (width 0.25) (layer F.Cu) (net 21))
 (via (at 78.4296 55.0034) (size 0.8) (drill 0.5) (layers F.Cu B.Cu) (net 21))
 (segment (start 80.0796 54.9974) (end 78.4356 54.9974) (width 0.25) (layer B.Cu) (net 21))
 (segment (start 78.4356 54.9974) (end 78.4296 55.0034) (width 0.25) (layer B.Cu) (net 21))
 (segment (start 83.4296 47.3534) (end 83.4296 49.2534) (width 0.35) (layer B.Cu) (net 20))
 (segment (start 83.4296 49.2534) (end 83.8796 49.7034) (width 0.35) (layer B.Cu) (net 20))
 (segment (start 83.8796 49.7034) (end 85.0796 49.7034) (width 0.35) (layer B.Cu) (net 20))
 (segment (start 83.4296 48.3699) (end 83.4296 47.3534) (width 0.35) (layer B.Cu) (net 20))
 (via (at 85.2796 51.1534) (size 0.8) (drill 0.5) (layers F.Cu B.Cu) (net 20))
 (segment (start 82.2631 48.3699) (end 83.4296 48.3699) (width 0.35) (layer B.Cu) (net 20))
 (segment (start 81.0346 48.3699) (end 82.2631 48.3699) (width 0.35) (layer B.Cu) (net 20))
 (segment (start 83.5496 48.3034) (end 84.6796 48.3034) (width 0.25) (layer F.Cu) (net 20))
 (segment (start 85.2796 48.9034) (end 85.2796 51.1534) (width 0.25) (layer F.Cu) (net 20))
 (segment (start 84.6796 48.3034) (end 85.2796 48.9034) (width 0.25) (layer F.Cu) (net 20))
 (segment (start 85.2796 49.9034) (end 85.0796 49.7034) (width 0.25) (layer B.Cu) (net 20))
 (segment (start 85.2796 51.1534) (end 85.2796 49.9034) (width 0.25) (layer B.Cu) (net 20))
 (segment (start 79.7646 49.6384) (end 79.7646 48.3699) (width 0.25) (layer B.Cu) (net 24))
 (segment (start 82.4296 49.8034) (end 79.9296 49.8034) (width 0.25) (layer B.Cu) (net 24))
 (segment (start 84.3796 51.7534) (end 82.4296 49.8034) (width 0.25) (layer B.Cu) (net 24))
 (segment (start 84.3796 53.6534) (end 84.3796 51.7534) (width 0.25) (layer B.Cu) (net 24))
 (segment (start 85.6796 54.9534) (end 84.3796 53.6534) (width 0.25) (layer B.Cu) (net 24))
 (segment (start 79.9296 49.8034) (end 79.7646 49.6384) (width 0.25) (layer B.Cu) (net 24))
 (segment (start 85.6796 54.9974) (end 85.6796 54.9534) (width 0.25) (layer B.Cu) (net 24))
 (segment (start 76.8796 54.8284) (end 76.7046 55.0034) (width 0.25) (layer B.Cu) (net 23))
 (segment (start 76.7046 54.0284) (end 76.7796 53.9534) (width 0.25) (layer B.Cu) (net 23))
 (segment (start 76.7046 55.0034) (end 76.7046 54.0284) (width 0.25) (layer B.Cu) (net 23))
 (via (at 76.7796 53.9534) (size 0.6) (drill 0.4) (layers F.Cu B.Cu) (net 23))
 (via (at 76.879582 50.1034) (size 0.6) (drill 0.4) (layers F.Cu B.Cu) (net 23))
 (segment (start 78.4946 49.3724) (end 77.7636 50.1034) (width 0.25) (layer B.Cu) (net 23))
 (segment (start 78.4946 48.3699) (end 78.4946 49.3724) (width 0.25) (layer B.Cu) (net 23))
 (segment (start 77.7636 50.1034) (end 76.879582 50.1034) (width 0.25) (layer B.Cu) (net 23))
 (segment (start 76.7796 53.9534) (end 76.7796 50.203382) (width 0.25) (layer F.Cu) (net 23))
 (segment (start 76.7796 50.203382) (end 76.879582 50.1034) (width 0.25) (layer F.Cu) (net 23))
 (segment (start 78.4946 41.318401) (end 78.479599 41.3034) (width 0.25) (layer B.Cu) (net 25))
 (segment (start 78.4946 43.3749) (end 78.4946 41.318401) (width 0.25) (layer B.Cu) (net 25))
 (segment (start 82.2796 45.3034) (end 81.548318 44.572118) (width 0.25) (layer F.Cu) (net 1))
 (segment (start 83.5496 45.3034) (end 82.2796 45.3034) (width 0.25) (layer F.Cu) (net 1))
 (segment (start 80.348318 44.572118) (end 81.548318 44.572118) (width 0.25) (layer F.Cu) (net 1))
 (segment (start 79.4796 44.0534) (end 79.8296 44.0534) (width 0.25) (layer F.Cu) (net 1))
 (segment (start 79.029949 44.503051) (end 79.4796 44.0534) (width 0.25) (layer F.Cu) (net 1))
 (segment (start 79.8296 44.0534) (end 80.348318 44.572118) (width 0.25) (layer F.Cu) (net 1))
 (segment (start 79.029949 44.506604) (end 79.029949 44.503051) (width 0.25) (layer F.Cu) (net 1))
 (segment (start 81.9296 47.1034) (end 82.2796 47.1034) (width 0.25) (layer F.Cu) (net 1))
 (segment (start 82.2796 45.3034) (end 82.2796 47.1034) (width 0.25) (layer F.Cu) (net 1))
 (segment (start 82.2796 49.9034) (end 81.9296 50.2534) (width 0.25) (layer F.Cu) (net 1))
 (segment (start 82.2796 47.1034) (end 82.2796 49.9034) (width 0.25) (layer F.Cu) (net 1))
 (via (at 81.6296 50.5534) (size 0.8) (drill 0.5) (layers F.Cu B.Cu) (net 1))
 (segment (start 81.9296 50.2534) (end 81.6296 50.5534) (width 0.25) (layer F.Cu) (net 1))
 (segment (start 73.079604 48.335629) (end 73.079604 49.2034) (width 0.25) (layer F.Cu) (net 1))
 (segment (start 74.522144 46.893089) (end 73.079604 48.335629) (width 0.25) (layer F.Cu) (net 1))
 (segment (start 74.829603 50.953399) (end 73.079604 49.2034) (width 0.25) (layer B.Cu) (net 1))
 (segment (start 81.229601 50.953399) (end 74.829603 50.953399) (width 0.25) (layer B.Cu) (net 1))
 (segment (start 81.6296 50.5534) (end 81.229601 50.953399) (width 0.25) (layer B.Cu) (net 1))
 (via (at 73.079604 49.2034) (size 0.8) (drill 0.5) (layers F.Cu B.Cu) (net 1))
 (segment (start 81.8296 54.9974) (end 83.9296 54.9974) (width 0.95) (layer B.Cu) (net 26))
 (segment (start 72.3546 55.0034) (end 74.9546 55.0034) (width 0.95) (layer B.Cu) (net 27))
 (segment (start 79.770589 48.340836) (end 80.692164 48.340836) (width 0.25) (layer F.Cu) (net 19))
 (segment (start 79.029949 47.600196) (end 79.770589 48.340836) (width 0.25) (layer F.Cu) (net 19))
 (segment (start 75.9961 48.3699) (end 75.4796 47.8534) (width 0.25) (layer B.Cu) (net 22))
 (segment (start 77.2246 48.3699) (end 75.9961 48.3699) (width 0.25) (layer B.Cu) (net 22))
 (segment (start 73.0977 51.853067) (end 73.0977 53.0502) (width 0.25) (layer F.Cu) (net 13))
 (segment (start 76.289911 48.660856) (end 73.0977 51.853067) (width 0.25) (layer F.Cu) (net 13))
 (segment (start 76.643464 49.01441) (end 76.643464 49.039536) (width 0.25) (layer F.Cu) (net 14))
 (segment (start 75.5977 50.0853) (end 75.5977 53.0502) (width 0.25) (layer F.Cu) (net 14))
 (segment (start 76.643464 49.039536) (end 75.5977 50.0853) (width 0.25) (layer F.Cu) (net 14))
 (segment (start 78.0796 53.0321) (end 78.0977 53.0502) (width 0.25) (layer F.Cu) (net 15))
 (segment (start 78.0796 49.478274) (end 78.0796 53.0321) (width 0.25) (layer F.Cu) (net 15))
 (segment (start 77.615736 49.01441) (end 78.0796 49.478274) (width 0.25) (layer F.Cu) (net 15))
 (segment (start 80.5764 53.0502) (end 80.5977 53.0502) (width 0.25) (layer F.Cu) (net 16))
 (segment (start 78.5796 51.0534) (end 80.5764 53.0502) (width 0.25) (layer F.Cu) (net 16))
 (segment (start 78.5796 49.2534) (end 78.5796 51.0534) (width 0.25) (layer F.Cu) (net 16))
 (segment (start 77.987056 48.660856) (end 78.5796 49.2534) (width 0.25) (layer F.Cu) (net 16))
 (segment (start 77.969289 48.660856) (end 77.987056 48.660856) (width 0.25) (layer F.Cu) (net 16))
 (segment (start 83.0764 53.0502) (end 83.0977 53.0502) (width 0.25) (layer F.Cu) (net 17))
 (segment (start 81.7796 51.7534) (end 83.0764 53.0502) (width 0.25) (layer F.Cu) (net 17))
 (segment (start 80.2296 51.7534) (end 81.7796 51.7534) (width 0.25) (layer F.Cu) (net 17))
 (segment (start 79.02961 50.55341) (end 80.2296 51.7534) (width 0.25) (layer F.Cu) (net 17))
 (segment (start 79.02961 49.067) (end 79.02961 50.55341) (width 0.25) (layer F.Cu) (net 17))
 (segment (start 78.322843 48.360233) (end 79.02961 49.067) (width 0.25) (layer F.Cu) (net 17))
 (segment (start 78.322843 48.307303) (end 78.322843 48.360233) (width 0.25) (layer F.Cu) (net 17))
 (segment (start 85.5977 53.0215) (end 85.5977 53.0502) (width 0.25) (layer F.Cu) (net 18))
 (segment (start 83.87959 51.30339) (end 85.5977 53.0215) (width 0.25) (layer F.Cu) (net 18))
 (segment (start 80.67959 51.30339) (end 83.87959 51.30339) (width 0.25) (layer F.Cu) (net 18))
 (segment (start 79.47962 48.8806) (end 79.47962 50.10342) (width 0.25) (layer F.Cu) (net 18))
 (segment (start 79.019712 48.420692) (end 79.47962 48.8806) (width 0.25) (layer F.Cu) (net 18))
 (segment (start 79.47962 50.10342) (end 80.67959 51.30339) (width 0.25) (layer F.Cu) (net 18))
 (segment (start 79.019712 48.367762) (end 79.019712 48.420692) (width 0.25) (layer F.Cu) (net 18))
 (segment (start 78.676396 48.024446) (end 79.019712 48.367762) (width 0.25) (layer F.Cu) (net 18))
 (segment (start 78.676396 47.953749) (end 78.676396 48.024446) (width 0.25) (layer F.Cu) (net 18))
 (segment (start 82.5945 42.0534) (end 85.5977 39.0502) (width 0.25) (layer F.Cu) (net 3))
 (segment (start 80.06894 42.0534) (end 82.5945 42.0534) (width 0.25) (layer F.Cu) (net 3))
 (segment (start 78.322843 43.799497) (end 80.06894 42.0534) (width 0.25) (layer F.Cu) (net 3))
 (segment (start 83.0977 40.2853) (end 83.0977 39.0502) (width 0.25) (layer F.Cu) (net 4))
 (segment (start 81.947357 41.435643) (end 83.0977 40.2853) (width 0.25) (layer F.Cu) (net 4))
 (segment (start 79.97959 41.435643) (end 81.947357 41.435643) (width 0.25) (layer F.Cu) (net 4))
 (segment (start 77.969289 43.445944) (end 79.97959 41.435643) (width 0.25) (layer F.Cu) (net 4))
 (segment (start 80.5796 39.0683) (end 80.5977 39.0502) (width 0.25) (layer F.Cu) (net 5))
 (segment (start 80.5796 40.1034) (end 80.5796 39.0683) (width 0.25) (layer F.Cu) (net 5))
 (segment (start 77.615736 43.067264) (end 80.5796 40.1034) (width 0.25) (layer F.Cu) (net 5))
 (segment (start 77.615736 43.09239) (end 77.615736 43.067264) (width 0.25) (layer F.Cu) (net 5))
 (segment (start 73.9296 39.8821) (end 73.0977 39.0502) (width 0.25) (layer F.Cu) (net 8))
 (segment (start 75.929094 43.799497) (end 73.9296 41.800003) (width 0.25) (layer F.Cu) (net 8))
 (segment (start 73.9296 41.800003) (end 73.9296 39.8821) (width 0.25) (layer F.Cu) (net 8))
 (segment (start 75.936357 43.799497) (end 75.929094 43.799497) (width 0.25) (layer F.Cu) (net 8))
 (segment (start 76.289911 43.445944) (end 76.272144 43.445944) (width 0.25) (layer F.Cu) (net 7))
 (segment (start 75.5977 42.7715) (end 75.5977 39.0502) (width 0.25) (layer F.Cu) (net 7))
 (segment (start 76.272144 43.445944) (end 75.5977 42.7715) (width 0.25) (layer F.Cu) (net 7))
 (segment (start 76.2296 42.0534) (end 78.0977 40.1853) (width 0.25) (layer F.Cu) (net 6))
 (segment (start 78.0977 40.1853) (end 78.0977 39.0502) (width 0.25) (layer F.Cu) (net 6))
 (segment (start 76.2296 42.7034) (end 76.2296 42.0534) (width 0.25) (layer F.Cu) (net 6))
 (segment (start 76.61859 43.09239) (end 76.2296 42.7034) (width 0.25) (layer F.Cu) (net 6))
 (segment (start 76.643464 43.09239) (end 76.61859 43.09239) (width 0.25) (layer F.Cu) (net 6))
 (segment (start 71.9445 51.7034) (end 70.5977 53.0502) (width 0.25) (layer F.Cu) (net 12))
 (segment (start 72.54026 51.7034) (end 71.9445 51.7034) (width 0.25) (layer F.Cu) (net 12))
 (segment (start 75.936357 48.307303) (end 72.54026 51.7034) (width 0.25) (layer F.Cu) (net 12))
 (segment (start 68.0977 51.6853) (end 68.0977 53.0502) (width 0.25) (layer F.Cu) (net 11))
 (segment (start 72.4296 51.1034) (end 68.6796 51.1034) (width 0.25) (layer F.Cu) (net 11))
 (segment (start 74.7796 48.7534) (end 72.4296 51.1034) (width 0.25) (layer F.Cu) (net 11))
 (segment (start 68.6796 51.1034) (end 68.0977 51.6853) (width 0.25) (layer F.Cu) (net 11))
 (segment (start 74.7796 48.049847) (end 74.7796 48.7534) (width 0.25) (layer F.Cu) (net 11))
 (segment (start 75.229251 47.600196) (end 74.7796 48.049847) (width 0.25) (layer F.Cu) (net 11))
 (segment (start 75.229251 44.506604) (end 71.726047 41.0034) (width 0.25) (layer F.Cu) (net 10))
 (segment (start 71.726047 41.0034) (end 68.6796 41.0034) (width 0.25) (layer F.Cu) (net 10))
 (segment (start 68.0977 40.4215) (end 68.0977 39.0502) (width 0.25) (layer F.Cu) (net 10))
 (segment (start 68.6796 41.0034) (end 68.0977 40.4215) (width 0.25) (layer F.Cu) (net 10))
 (segment (start 70.5977 39.1715) (end 70.5977 39.0502) (width 0.25) (layer F.Cu) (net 9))
 (segment (start 75.579251 44.153051) (end 70.5977 39.1715) (width 0.25) (layer F.Cu) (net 9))
 (segment (start 75.582804 44.153051) (end 75.579251 44.153051) (width 0.25) (layer F.Cu) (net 9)))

